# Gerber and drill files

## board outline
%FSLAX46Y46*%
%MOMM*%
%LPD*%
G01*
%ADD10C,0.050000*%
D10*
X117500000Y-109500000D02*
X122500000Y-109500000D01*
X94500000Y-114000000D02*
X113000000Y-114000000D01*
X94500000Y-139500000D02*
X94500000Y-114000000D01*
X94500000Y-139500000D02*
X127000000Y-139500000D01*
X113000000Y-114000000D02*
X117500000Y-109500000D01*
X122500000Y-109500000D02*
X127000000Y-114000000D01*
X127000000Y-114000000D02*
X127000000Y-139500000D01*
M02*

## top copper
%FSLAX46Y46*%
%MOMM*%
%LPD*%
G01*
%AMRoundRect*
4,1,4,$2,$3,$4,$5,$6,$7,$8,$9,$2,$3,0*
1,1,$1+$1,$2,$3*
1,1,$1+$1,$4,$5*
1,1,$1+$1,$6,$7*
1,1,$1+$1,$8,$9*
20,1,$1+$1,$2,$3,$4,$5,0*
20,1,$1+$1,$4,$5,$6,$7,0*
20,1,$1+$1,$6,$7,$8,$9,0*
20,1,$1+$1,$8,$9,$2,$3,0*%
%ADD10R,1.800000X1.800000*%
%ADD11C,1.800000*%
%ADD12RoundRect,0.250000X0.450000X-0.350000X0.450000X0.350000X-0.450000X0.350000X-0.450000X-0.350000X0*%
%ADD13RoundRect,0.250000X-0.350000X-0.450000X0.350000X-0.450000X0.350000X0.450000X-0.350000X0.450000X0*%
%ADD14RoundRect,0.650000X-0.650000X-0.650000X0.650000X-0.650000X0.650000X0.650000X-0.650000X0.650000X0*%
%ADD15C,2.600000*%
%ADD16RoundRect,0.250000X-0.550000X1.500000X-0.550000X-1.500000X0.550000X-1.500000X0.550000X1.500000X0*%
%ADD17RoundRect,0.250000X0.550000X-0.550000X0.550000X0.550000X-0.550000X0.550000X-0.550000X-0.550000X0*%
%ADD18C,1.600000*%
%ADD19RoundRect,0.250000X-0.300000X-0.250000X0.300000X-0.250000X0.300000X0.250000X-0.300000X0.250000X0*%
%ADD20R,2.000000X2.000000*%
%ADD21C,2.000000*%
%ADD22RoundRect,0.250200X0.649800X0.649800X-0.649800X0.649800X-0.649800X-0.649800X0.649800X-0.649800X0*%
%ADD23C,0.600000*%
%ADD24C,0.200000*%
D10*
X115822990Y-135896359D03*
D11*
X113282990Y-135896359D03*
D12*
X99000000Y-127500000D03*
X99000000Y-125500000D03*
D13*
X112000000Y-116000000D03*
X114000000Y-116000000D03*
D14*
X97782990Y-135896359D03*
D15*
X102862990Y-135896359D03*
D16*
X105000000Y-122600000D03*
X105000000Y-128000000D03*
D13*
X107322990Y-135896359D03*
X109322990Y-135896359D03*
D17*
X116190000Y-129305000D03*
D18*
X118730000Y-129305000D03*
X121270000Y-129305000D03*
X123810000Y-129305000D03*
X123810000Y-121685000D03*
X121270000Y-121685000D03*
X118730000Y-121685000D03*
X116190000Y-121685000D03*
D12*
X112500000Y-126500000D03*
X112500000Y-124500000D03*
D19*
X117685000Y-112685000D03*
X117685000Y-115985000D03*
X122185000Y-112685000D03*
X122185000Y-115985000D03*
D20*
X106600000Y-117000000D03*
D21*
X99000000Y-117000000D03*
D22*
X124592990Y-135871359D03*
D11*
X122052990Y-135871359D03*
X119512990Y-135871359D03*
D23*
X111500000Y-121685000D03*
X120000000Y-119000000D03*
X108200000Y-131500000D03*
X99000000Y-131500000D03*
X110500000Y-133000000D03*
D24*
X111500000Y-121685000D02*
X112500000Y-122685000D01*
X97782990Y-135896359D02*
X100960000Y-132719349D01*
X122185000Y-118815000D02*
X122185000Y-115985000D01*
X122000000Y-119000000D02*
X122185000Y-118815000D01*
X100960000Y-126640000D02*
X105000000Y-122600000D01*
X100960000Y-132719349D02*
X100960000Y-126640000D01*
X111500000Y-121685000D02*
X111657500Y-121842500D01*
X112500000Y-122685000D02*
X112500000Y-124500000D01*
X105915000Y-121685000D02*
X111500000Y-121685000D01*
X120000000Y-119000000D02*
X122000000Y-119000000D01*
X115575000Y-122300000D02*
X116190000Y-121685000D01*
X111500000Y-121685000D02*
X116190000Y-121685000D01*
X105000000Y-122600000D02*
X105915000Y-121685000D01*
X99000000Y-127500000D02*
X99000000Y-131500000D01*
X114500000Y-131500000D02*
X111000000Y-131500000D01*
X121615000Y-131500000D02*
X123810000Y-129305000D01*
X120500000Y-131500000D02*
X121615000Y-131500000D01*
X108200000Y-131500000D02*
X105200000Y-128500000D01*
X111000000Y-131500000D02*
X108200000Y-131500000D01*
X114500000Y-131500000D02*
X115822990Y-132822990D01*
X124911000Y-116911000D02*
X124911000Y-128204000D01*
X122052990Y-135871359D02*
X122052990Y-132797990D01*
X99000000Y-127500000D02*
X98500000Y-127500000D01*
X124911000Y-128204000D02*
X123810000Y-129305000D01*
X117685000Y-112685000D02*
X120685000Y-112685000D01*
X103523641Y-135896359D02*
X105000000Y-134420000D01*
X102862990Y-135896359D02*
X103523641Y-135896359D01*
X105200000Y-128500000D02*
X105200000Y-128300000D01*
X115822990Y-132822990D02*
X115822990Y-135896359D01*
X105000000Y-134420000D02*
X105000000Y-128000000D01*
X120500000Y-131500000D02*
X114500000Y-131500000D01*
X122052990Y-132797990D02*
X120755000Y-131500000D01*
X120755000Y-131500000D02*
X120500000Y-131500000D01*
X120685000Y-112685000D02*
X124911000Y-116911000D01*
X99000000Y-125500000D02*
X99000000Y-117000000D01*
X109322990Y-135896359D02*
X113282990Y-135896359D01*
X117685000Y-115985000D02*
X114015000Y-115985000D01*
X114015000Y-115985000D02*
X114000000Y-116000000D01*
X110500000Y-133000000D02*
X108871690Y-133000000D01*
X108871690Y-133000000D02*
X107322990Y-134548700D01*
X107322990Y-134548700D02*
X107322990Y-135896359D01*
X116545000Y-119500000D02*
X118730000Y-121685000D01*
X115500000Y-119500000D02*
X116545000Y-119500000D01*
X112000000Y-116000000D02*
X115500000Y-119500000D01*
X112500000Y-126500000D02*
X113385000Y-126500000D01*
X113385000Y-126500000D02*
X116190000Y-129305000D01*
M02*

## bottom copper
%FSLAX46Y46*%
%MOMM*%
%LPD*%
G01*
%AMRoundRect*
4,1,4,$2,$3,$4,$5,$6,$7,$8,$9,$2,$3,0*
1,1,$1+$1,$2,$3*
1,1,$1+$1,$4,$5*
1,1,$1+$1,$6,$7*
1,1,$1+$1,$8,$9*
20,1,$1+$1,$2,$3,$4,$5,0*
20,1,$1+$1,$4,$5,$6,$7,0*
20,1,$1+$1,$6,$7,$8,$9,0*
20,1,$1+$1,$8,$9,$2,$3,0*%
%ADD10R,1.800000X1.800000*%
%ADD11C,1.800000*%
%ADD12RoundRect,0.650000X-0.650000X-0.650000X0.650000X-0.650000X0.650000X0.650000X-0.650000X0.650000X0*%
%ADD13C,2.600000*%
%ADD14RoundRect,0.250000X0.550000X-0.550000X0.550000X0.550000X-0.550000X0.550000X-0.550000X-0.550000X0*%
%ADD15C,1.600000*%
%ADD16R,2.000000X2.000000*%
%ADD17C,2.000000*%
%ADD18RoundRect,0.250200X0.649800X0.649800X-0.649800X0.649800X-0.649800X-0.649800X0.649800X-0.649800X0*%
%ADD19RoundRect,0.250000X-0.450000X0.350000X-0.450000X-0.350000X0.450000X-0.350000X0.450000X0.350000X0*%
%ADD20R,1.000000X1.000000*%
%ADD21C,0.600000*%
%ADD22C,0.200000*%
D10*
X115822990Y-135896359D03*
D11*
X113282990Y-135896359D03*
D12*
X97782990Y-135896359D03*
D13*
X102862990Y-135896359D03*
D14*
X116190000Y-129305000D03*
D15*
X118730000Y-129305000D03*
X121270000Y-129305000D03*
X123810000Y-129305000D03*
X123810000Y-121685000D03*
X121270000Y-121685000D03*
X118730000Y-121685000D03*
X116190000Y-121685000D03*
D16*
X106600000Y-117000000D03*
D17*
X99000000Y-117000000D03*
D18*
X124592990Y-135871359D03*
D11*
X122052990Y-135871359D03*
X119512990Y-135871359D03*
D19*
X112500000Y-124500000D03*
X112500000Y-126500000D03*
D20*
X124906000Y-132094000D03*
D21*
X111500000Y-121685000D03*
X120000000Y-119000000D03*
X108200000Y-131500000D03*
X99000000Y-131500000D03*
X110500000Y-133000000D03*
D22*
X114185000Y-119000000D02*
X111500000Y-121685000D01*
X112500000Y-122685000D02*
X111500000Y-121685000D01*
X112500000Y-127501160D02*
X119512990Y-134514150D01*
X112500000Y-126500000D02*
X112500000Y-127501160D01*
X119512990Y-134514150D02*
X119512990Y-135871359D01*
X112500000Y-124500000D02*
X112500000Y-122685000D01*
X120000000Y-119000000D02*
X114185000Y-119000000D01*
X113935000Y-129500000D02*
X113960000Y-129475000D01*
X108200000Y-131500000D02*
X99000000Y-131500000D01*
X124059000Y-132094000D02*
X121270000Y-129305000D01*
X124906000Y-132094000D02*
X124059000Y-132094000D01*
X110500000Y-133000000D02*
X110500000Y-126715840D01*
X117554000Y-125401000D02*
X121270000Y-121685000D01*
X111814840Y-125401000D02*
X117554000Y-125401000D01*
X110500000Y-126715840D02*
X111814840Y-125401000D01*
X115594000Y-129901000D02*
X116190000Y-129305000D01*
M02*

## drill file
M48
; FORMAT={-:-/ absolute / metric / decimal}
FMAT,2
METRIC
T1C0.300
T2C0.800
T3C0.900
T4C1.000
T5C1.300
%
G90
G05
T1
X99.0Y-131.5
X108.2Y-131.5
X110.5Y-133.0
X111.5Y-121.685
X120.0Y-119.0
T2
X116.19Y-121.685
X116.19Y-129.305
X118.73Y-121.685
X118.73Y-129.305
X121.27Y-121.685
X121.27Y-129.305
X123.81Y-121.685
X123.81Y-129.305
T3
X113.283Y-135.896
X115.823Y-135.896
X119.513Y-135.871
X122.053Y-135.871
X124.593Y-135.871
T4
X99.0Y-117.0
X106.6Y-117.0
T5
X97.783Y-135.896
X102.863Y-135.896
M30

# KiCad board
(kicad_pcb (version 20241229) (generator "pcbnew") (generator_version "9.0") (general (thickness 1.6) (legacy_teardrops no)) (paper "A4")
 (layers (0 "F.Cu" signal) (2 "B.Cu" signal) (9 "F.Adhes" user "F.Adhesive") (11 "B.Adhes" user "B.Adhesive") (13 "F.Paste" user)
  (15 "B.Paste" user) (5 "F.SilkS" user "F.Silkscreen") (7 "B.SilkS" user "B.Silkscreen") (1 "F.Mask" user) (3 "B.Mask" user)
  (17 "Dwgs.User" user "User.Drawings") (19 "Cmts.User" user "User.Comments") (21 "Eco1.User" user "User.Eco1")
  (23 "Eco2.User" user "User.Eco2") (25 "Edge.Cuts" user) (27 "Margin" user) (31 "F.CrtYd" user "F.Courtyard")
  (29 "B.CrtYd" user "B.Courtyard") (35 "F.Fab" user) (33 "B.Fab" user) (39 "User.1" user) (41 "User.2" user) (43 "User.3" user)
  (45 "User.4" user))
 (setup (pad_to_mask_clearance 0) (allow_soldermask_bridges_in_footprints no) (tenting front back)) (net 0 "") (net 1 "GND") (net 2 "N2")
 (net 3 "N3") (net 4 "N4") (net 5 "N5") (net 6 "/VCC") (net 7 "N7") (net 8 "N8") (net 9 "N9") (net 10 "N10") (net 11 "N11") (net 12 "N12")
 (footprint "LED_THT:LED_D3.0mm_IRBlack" (layer "F.Cu") (at 115.82299 135.896359 180)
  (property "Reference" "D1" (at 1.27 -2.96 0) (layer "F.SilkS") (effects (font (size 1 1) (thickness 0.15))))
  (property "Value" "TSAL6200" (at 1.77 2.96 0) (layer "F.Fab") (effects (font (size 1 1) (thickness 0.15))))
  (pad "1" thru_hole rect (at 0 0 180) (size 1.8 1.8) (drill 0.9) (layers "*.Cu" "*.Mask") (remove_unused_layers no) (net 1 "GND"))
  (pad "2" thru_hole circle (at 2.54 0 180) (size 1.8 1.8) (drill 0.9) (layers "*.Cu" "*.Mask") (remove_unused_layers no) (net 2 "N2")))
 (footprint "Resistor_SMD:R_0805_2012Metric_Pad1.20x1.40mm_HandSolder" (layer "F.Cu") (at 99 126.5 90)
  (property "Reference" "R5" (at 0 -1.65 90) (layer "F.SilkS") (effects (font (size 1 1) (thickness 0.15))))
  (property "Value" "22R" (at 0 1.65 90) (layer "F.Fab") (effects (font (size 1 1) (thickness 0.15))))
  (pad "1" smd roundrect (at -1 0 90) (size 1.2 1.4) (layers "F.Cu" "F.Mask" "F.Paste") (roundrect_rratio 0.208333) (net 1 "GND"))
  (pad "2" smd roundrect (at 1 0 90) (size 1.2 1.4) (layers "F.Cu" "F.Mask" "F.Paste") (roundrect_rratio 0.208333) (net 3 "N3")))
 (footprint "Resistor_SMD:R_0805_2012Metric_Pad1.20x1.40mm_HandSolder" (layer "F.Cu") (at 113 116)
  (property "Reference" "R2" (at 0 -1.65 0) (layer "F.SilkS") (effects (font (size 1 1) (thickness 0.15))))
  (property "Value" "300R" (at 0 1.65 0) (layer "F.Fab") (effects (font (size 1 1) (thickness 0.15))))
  (pad "1" smd roundrect (at -1 0) (size 1.2 1.4) (layers "F.Cu" "F.Mask" "F.Paste") (roundrect_rratio 0.208333) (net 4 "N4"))
  (pad "2" smd roundrect (at 1 0) (size 1.2 1.4) (layers "F.Cu" "F.Mask" "F.Paste") (roundrect_rratio 0.208333) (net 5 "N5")))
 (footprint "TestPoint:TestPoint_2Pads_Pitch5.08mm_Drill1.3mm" (layer "F.Cu") (at 97.78299 135.896359)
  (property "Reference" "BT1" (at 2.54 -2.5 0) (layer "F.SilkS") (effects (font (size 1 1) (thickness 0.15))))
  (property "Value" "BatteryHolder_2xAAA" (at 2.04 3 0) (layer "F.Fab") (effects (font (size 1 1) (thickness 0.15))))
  (pad "1" thru_hole roundrect (at 0 0) (size 2.6 2.6) (drill 1.3) (layers "*.Cu" "*.Mask") (remove_unused_layers no)
   (roundrect_rratio 0.25) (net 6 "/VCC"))
  (pad "2" thru_hole circle (at 5.08 0) (size 2.6 2.6) (drill 1.3) (layers "*.Cu" "*.Mask") (remove_unused_layers no) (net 1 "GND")))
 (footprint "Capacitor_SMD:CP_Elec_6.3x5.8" (layer "F.Cu") (at 105 125.3 -90)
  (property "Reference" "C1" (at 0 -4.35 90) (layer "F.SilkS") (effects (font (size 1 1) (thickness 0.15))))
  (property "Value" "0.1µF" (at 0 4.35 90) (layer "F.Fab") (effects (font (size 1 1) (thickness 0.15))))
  (pad "1" smd roundrect (at -2.7 0 270) (size 3.5 1.6) (layers "F.Cu" "F.Mask" "F.Paste") (roundrect_rratio 0.15625) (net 6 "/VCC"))
  (pad "2" smd roundrect (at 2.7 0 270) (size 3.5 1.6) (layers "F.Cu" "F.Mask" "F.Paste") (roundrect_rratio 0.15625) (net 1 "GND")))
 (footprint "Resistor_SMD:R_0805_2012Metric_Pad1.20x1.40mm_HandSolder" (layer "F.Cu") (at 108.32299 135.896359)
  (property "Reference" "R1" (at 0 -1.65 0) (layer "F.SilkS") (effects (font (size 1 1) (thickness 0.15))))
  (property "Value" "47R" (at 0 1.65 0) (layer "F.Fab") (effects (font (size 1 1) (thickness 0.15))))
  (pad "1" smd roundrect (at -1 0) (size 1.2 1.4) (layers "F.Cu" "F.Mask" "F.Paste") (roundrect_rratio 0.208333) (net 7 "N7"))
  (pad "2" smd roundrect (at 1 0) (size 1.2 1.4) (layers "F.Cu" "F.Mask" "F.Paste") (roundrect_rratio 0.208333) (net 2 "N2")))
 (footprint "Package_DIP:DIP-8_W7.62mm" (layer "F.Cu") (at 116.19 129.305 90)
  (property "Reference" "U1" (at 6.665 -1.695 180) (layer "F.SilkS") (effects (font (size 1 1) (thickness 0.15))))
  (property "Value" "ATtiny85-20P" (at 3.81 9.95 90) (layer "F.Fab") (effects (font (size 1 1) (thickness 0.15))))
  (pad "1" thru_hole roundrect (at 0 0 90) (size 1.6 1.6) (drill 0.8) (layers "*.Cu" "*.Mask") (remove_unused_layers no)
   (roundrect_rratio 0.15625) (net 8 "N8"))
  (pad "2" thru_hole circle (at 0 2.54 90) (size 1.6 1.6) (drill 0.8) (layers "*.Cu" "*.Mask") (remove_unused_layers no) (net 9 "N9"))
  (pad "3" thru_hole circle (at 0 5.08 90) (size 1.6 1.6) (drill 0.8) (layers "*.Cu" "*.Mask") (remove_unused_layers no) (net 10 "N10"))
  (pad "4" thru_hole circle (at 0 7.62 90) (size 1.6 1.6) (drill 0.8) (layers "*.Cu" "*.Mask") (remove_unused_layers no) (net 1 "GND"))
  (pad "5" thru_hole circle (at 7.62 7.62 90) (size 1.6 1.6) (drill 0.8) (layers "*.Cu" "*.Mask") (remove_unused_layers no) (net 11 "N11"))
  (pad "6" thru_hole circle (at 7.62 5.08 90) (size 1.6 1.6) (drill 0.8) (layers "*.Cu" "*.Mask") (remove_unused_layers no) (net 7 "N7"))
  (pad "7" thru_hole circle (at 7.62 2.54 90) (size 1.6 1.6) (drill 0.8) (layers "*.Cu" "*.Mask") (remove_unused_layers no) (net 4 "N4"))
  (pad "8" thru_hole circle (at 7.62 0 90) (size 1.6 1.6) (drill 0.8) (layers "*.Cu" "*.Mask") (remove_unused_layers no) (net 6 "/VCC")))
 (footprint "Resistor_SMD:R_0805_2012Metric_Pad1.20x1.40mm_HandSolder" (layer "F.Cu") (at 112.5 125.5 90)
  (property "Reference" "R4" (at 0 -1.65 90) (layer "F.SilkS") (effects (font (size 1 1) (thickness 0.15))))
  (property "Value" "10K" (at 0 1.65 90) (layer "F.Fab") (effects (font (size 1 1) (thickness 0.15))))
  (pad "1" smd roundrect (at -1 0 90) (size 1.2 1.4) (layers "F.Cu" "F.Mask" "F.Paste") (roundrect_rratio 0.208333) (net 8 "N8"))
  (pad "2" smd roundrect (at 1 0 90) (size 1.2 1.4) (layers "F.Cu" "F.Mask" "F.Paste") (roundrect_rratio 0.208333) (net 6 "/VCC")))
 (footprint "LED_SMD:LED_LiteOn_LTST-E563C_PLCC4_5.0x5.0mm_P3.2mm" (layer "F.Cu") (at 119.935 114.335)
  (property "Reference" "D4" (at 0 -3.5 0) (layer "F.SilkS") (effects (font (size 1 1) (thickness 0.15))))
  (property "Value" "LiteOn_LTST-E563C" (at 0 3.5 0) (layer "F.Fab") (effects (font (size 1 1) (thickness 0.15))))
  (pad "1" smd roundrect (at -2.25 -1.65) (size 1.1 1) (layers "F.Cu" "F.Mask" "F.Paste") (roundrect_rratio 0.25) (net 1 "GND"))
  (pad "2" smd roundrect (at -2.25 1.65) (size 1.1 1) (layers "F.Cu" "F.Mask" "F.Paste") (roundrect_rratio 0.25) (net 5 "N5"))
  (pad "3" smd roundrect (at 2.25 -1.65) (size 1.1 1) (layers "F.Cu" "F.Mask" "F.Paste") (roundrect_rratio 0.25) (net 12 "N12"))
  (pad "4" smd roundrect (at 2.25 1.65) (size 1.1 1) (layers "F.Cu" "F.Mask" "F.Paste") (roundrect_rratio 0.25) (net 6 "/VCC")))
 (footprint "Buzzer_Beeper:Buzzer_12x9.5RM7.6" (layer "B.Cu") (at 106.6 117 180)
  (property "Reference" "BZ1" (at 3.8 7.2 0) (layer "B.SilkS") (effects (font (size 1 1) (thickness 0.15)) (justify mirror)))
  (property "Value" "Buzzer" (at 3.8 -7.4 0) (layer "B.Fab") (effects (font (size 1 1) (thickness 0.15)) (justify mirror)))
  (pad "1" thru_hole rect (at 0 0 180) (size 2 2) (drill 1) (layers "*.Cu" "*.Mask") (remove_unused_layers no) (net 9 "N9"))
  (pad "2" thru_hole circle (at 7.6 0 180) (size 2 2) (drill 1) (layers "*.Cu" "*.Mask") (remove_unused_layers no) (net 3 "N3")))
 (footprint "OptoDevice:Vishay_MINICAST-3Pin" (layer "B.Cu") (at 124.59299 135.871359 180)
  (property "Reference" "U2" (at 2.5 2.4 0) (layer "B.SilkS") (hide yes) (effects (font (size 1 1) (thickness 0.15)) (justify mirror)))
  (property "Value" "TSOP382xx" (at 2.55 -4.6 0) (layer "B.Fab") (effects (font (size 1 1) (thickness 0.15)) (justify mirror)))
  (pad "1" thru_hole roundrect (at 0 0 180) (size 1.8 1.8) (drill 0.9) (layers "*.Cu" "*.Mask") (remove_unused_layers no)
   (roundrect_rratio 0.139) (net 11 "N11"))
  (pad "2" thru_hole circle (at 2.54 0 180) (size 1.8 1.8) (drill 0.9) (layers "*.Cu" "*.Mask") (remove_unused_layers no) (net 1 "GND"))
  (pad "3" thru_hole circle (at 5.08 0 180) (size 1.8 1.8) (drill 0.9) (layers "*.Cu" "*.Mask") (remove_unused_layers no) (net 6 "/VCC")))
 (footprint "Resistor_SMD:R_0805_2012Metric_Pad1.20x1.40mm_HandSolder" (layer "B.Cu") (at 112.5 125.5 -90)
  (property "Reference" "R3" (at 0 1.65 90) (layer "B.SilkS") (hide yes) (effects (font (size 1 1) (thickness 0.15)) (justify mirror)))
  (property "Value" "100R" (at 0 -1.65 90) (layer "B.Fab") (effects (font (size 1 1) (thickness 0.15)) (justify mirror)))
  (pad "1" smd roundrect (at -1 0 270) (size 1.2 1.4) (layers "B.Cu" "B.Mask" "B.Paste") (roundrect_rratio 0.208333) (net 6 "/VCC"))
  (pad "2" smd roundrect (at 1 0 270) (size 1.2 1.4) (layers "B.Cu" "B.Mask" "B.Paste") (roundrect_rratio 0.208333) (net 6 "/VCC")))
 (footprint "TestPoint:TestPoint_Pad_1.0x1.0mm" (layer "B.Cu") (at 124.906 132.094 180)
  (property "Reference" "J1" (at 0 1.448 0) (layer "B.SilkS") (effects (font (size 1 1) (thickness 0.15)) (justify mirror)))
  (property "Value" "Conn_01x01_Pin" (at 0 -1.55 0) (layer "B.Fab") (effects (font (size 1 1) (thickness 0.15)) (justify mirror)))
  (pad "1" smd rect (at 0 0 180) (size 1 1) (layers "B.Cu" "B.Mask") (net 10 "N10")))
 (gr_line (start 117.5 109.5) (end 122.5 109.5) (stroke (width 0.05) (type default)) (layer "Edge.Cuts"))
 (gr_line (start 94.5 114) (end 113 114) (stroke (width 0.05) (type default)) (layer "Edge.Cuts"))
 (gr_line (start 94.5 139.5) (end 94.5 114) (stroke (width 0.05) (type default)) (layer "Edge.Cuts"))
 (gr_line (start 94.5 139.5) (end 127 139.5) (stroke (width 0.05) (type default)) (layer "Edge.Cuts"))
 (gr_line (start 113 114) (end 117.5 109.5) (stroke (width 0.05) (type default)) (layer "Edge.Cuts"))
 (gr_line (start 122.5 109.5) (end 127 114) (stroke (width 0.05) (type default)) (layer "Edge.Cuts"))
 (gr_line (start 127 114) (end 127 139.5) (stroke (width 0.05) (type default)) (layer "Edge.Cuts"))
 (segment (start 111.5 121.685) (end 112.5 122.685) (width 0.2) (layer "F.Cu") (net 6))
 (segment (start 97.78299 135.896359) (end 100.96 132.719349) (width 0.2) (layer "F.Cu") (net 6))
 (segment (start 122.185 118.815) (end 122.185 115.985) (width 0.2) (layer "F.Cu") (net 6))
 (segment (start 122 119) (end 122.185 118.815) (width 0.2) (layer "F.Cu") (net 6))
 (segment (start 100.96 126.64) (end 105 122.6) (width 0.2) (layer "F.Cu") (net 6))
 (segment (start 100.96 132.719349) (end 100.96 126.64) (width 0.2) (layer "F.Cu") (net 6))
 (segment (start 111.5 121.685) (end 111.6575 121.8425) (width 0.2) (layer "F.Cu") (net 6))
 (segment (start 112.5 122.685) (end 112.5 124.5) (width 0.2) (layer "F.Cu") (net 6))
 (segment (start 105.915 121.685) (end 111.5 121.685) (width 0.2) (layer "F.Cu") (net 6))
 (segment (start 120 119) (end 122 119) (width 0.2) (layer "F.Cu") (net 6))
 (segment (start 115.575 122.3) (end 116.19 121.685) (width 0.2) (layer "F.Cu") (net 6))
 (segment (start 111.5 121.685) (end 116.19 121.685) (width 0.2) (layer "F.Cu") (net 6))
 (segment (start 105 122.6) (end 105.915 121.685) (width 0.2) (layer "F.Cu") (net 6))
 (via (at 111.5 121.685) (size 0.6) (drill 0.3) (layers "F.Cu" "B.Cu") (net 6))
 (via (at 120 119) (size 0.6) (drill 0.3) (layers "F.Cu" "B.Cu") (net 6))
 (segment (start 114.185 119) (end 111.5 121.685) (width 0.2) (layer "B.Cu") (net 6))
 (segment (start 112.5 122.685) (end 111.5 121.685) (width 0.2) (layer "B.Cu") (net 6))
 (segment (start 112.5 127.50116) (end 119.51299 134.51415) (width 0.2) (layer "B.Cu") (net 6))
 (segment (start 112.5 126.5) (end 112.5 127.50116) (width 0.2) (layer "B.Cu") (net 6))
 (segment (start 119.51299 134.51415) (end 119.51299 135.871359) (width 0.2) (layer "B.Cu") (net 6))
 (segment (start 112.5 124.5) (end 112.5 122.685) (width 0.2) (layer "B.Cu") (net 6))
 (segment (start 120 119) (end 114.185 119) (width 0.2) (layer "B.Cu") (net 6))
 (segment (start 113.935 129.5) (end 113.96 129.475) (width 0.2) (layer "B.Cu") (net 6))
 (segment (start 99 127.5) (end 99 131.5) (width 0.2) (layer "F.Cu") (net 1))
 (segment (start 114.5 131.5) (end 111 131.5) (width 0.2) (layer "F.Cu") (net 1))
 (segment (start 121.615 131.5) (end 123.81 129.305) (width 0.2) (layer "F.Cu") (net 1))
 (segment (start 120.5 131.5) (end 121.615 131.5) (width 0.2) (layer "F.Cu") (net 1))
 (segment (start 108.2 131.5) (end 105.2 128.5) (width 0.2) (layer "F.Cu") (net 1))
 (segment (start 111 131.5) (end 108.2 131.5) (width 0.2) (layer "F.Cu") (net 1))
 (segment (start 114.5 131.5) (end 115.82299 132.82299) (width 0.2) (layer "F.Cu") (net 1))
 (segment (start 124.911 116.911) (end 124.911 128.204) (width 0.2) (layer "F.Cu") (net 1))
 (segment (start 122.05299 135.871359) (end 122.05299 132.79799) (width 0.2) (layer "F.Cu") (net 1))
 (segment (start 99 127.5) (end 98.5 127.5) (width 0.2) (layer "F.Cu") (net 1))
 (segment (start 124.911 128.204) (end 123.81 129.305) (width 0.2) (layer "F.Cu") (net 1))
 (segment (start 117.685 112.685) (end 120.685 112.685) (width 0.2) (layer "F.Cu") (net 1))
 (segment (start 103.523641 135.896359) (end 105 134.42) (width 0.2) (layer "F.Cu") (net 1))
 (segment (start 102.86299 135.896359) (end 103.523641 135.896359) (width 0.2) (layer "F.Cu") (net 1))
 (segment (start 105.2 128.5) (end 105.2 128.3) (width 0.2) (layer "F.Cu") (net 1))
 (segment (start 115.82299 132.82299) (end 115.82299 135.896359) (width 0.2) (layer "F.Cu") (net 1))
 (segment (start 105 134.42) (end 105 128) (width 0.2) (layer "F.Cu") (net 1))
 (segment (start 120.5 131.5) (end 114.5 131.5) (width 0.2) (layer "F.Cu") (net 1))
 (segment (start 122.05299 132.79799) (end 120.755 131.5) (width 0.2) (layer "F.Cu") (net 1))
 (segment (start 120.755 131.5) (end 120.5 131.5) (width 0.2) (layer "F.Cu") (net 1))
 (segment (start 120.685 112.685) (end 124.911 116.911) (width 0.2) (layer "F.Cu") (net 1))
 (via (at 108.2 131.5) (size 0.6) (drill 0.3) (layers "F.Cu" "B.Cu") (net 1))
 (via (at 99 131.5) (size 0.6) (drill 0.3) (layers "F.Cu" "B.Cu") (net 1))
 (segment (start 108.2 131.5) (end 99 131.5) (width 0.2) (layer "B.Cu") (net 1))
 (segment (start 99 125.5) (end 99 117) (width 0.2) (layer "F.Cu") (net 3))
 (segment (start 109.32299 135.896359) (end 113.28299 135.896359) (width 0.2) (layer "F.Cu") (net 2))
 (segment (start 117.685 115.985) (end 114.015 115.985) (width 0.2) (layer "F.Cu") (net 5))
 (segment (start 114.015 115.985) (end 114 116) (width 0.2) (layer "F.Cu") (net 5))
 (segment (start 124.059 132.094) (end 121.27 129.305) (width 0.2) (layer "B.Cu") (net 10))
 (segment (start 124.906 132.094) (end 124.059 132.094) (width 0.2) (layer "B.Cu") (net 10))
 (segment (start 110.5 133) (end 108.87169 133) (width 0.2) (layer "F.Cu") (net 7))
 (segment (start 108.87169 133) (end 107.32299 134.5487) (width 0.2) (layer "F.Cu") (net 7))
 (segment (start 107.32299 134.5487) (end 107.32299 135.896359) (width 0.2) (layer "F.Cu") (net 7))
 (via (at 110.5 133) (size 0.6) (drill 0.3) (layers "F.Cu" "B.Cu") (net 7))
 (segment (start 110.5 133) (end 110.5 126.71584) (width 0.2) (layer "B.Cu") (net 7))
 (segment (start 117.554 125.401) (end 121.27 121.685) (width 0.2) (layer "B.Cu") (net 7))
 (segment (start 111.81484 125.401) (end 117.554 125.401) (width 0.2) (layer "B.Cu") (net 7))
 (segment (start 110.5 126.71584) (end 111.81484 125.401) (width 0.2) (layer "B.Cu") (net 7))
 (segment (start 116.545 119.5) (end 118.73 121.685) (width 0.2) (layer "F.Cu") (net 4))
 (segment (start 115.5 119.5) (end 116.545 119.5) (width 0.2) (layer "F.Cu") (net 4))
 (segment (start 112 116) (end 115.5 119.5) (width 0.2) (layer "F.Cu") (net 4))
 (segment (start 112.5 126.5) (end 113.385 126.5) (width 0.2) (layer "F.Cu") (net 8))
 (segment (start 113.385 126.5) (end 116.19 129.305) (width 0.2) (layer "F.Cu") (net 8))
 (segment (start 115.594 129.901) (end 116.19 129.305) (width 0.2) (layer "B.Cu") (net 8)))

